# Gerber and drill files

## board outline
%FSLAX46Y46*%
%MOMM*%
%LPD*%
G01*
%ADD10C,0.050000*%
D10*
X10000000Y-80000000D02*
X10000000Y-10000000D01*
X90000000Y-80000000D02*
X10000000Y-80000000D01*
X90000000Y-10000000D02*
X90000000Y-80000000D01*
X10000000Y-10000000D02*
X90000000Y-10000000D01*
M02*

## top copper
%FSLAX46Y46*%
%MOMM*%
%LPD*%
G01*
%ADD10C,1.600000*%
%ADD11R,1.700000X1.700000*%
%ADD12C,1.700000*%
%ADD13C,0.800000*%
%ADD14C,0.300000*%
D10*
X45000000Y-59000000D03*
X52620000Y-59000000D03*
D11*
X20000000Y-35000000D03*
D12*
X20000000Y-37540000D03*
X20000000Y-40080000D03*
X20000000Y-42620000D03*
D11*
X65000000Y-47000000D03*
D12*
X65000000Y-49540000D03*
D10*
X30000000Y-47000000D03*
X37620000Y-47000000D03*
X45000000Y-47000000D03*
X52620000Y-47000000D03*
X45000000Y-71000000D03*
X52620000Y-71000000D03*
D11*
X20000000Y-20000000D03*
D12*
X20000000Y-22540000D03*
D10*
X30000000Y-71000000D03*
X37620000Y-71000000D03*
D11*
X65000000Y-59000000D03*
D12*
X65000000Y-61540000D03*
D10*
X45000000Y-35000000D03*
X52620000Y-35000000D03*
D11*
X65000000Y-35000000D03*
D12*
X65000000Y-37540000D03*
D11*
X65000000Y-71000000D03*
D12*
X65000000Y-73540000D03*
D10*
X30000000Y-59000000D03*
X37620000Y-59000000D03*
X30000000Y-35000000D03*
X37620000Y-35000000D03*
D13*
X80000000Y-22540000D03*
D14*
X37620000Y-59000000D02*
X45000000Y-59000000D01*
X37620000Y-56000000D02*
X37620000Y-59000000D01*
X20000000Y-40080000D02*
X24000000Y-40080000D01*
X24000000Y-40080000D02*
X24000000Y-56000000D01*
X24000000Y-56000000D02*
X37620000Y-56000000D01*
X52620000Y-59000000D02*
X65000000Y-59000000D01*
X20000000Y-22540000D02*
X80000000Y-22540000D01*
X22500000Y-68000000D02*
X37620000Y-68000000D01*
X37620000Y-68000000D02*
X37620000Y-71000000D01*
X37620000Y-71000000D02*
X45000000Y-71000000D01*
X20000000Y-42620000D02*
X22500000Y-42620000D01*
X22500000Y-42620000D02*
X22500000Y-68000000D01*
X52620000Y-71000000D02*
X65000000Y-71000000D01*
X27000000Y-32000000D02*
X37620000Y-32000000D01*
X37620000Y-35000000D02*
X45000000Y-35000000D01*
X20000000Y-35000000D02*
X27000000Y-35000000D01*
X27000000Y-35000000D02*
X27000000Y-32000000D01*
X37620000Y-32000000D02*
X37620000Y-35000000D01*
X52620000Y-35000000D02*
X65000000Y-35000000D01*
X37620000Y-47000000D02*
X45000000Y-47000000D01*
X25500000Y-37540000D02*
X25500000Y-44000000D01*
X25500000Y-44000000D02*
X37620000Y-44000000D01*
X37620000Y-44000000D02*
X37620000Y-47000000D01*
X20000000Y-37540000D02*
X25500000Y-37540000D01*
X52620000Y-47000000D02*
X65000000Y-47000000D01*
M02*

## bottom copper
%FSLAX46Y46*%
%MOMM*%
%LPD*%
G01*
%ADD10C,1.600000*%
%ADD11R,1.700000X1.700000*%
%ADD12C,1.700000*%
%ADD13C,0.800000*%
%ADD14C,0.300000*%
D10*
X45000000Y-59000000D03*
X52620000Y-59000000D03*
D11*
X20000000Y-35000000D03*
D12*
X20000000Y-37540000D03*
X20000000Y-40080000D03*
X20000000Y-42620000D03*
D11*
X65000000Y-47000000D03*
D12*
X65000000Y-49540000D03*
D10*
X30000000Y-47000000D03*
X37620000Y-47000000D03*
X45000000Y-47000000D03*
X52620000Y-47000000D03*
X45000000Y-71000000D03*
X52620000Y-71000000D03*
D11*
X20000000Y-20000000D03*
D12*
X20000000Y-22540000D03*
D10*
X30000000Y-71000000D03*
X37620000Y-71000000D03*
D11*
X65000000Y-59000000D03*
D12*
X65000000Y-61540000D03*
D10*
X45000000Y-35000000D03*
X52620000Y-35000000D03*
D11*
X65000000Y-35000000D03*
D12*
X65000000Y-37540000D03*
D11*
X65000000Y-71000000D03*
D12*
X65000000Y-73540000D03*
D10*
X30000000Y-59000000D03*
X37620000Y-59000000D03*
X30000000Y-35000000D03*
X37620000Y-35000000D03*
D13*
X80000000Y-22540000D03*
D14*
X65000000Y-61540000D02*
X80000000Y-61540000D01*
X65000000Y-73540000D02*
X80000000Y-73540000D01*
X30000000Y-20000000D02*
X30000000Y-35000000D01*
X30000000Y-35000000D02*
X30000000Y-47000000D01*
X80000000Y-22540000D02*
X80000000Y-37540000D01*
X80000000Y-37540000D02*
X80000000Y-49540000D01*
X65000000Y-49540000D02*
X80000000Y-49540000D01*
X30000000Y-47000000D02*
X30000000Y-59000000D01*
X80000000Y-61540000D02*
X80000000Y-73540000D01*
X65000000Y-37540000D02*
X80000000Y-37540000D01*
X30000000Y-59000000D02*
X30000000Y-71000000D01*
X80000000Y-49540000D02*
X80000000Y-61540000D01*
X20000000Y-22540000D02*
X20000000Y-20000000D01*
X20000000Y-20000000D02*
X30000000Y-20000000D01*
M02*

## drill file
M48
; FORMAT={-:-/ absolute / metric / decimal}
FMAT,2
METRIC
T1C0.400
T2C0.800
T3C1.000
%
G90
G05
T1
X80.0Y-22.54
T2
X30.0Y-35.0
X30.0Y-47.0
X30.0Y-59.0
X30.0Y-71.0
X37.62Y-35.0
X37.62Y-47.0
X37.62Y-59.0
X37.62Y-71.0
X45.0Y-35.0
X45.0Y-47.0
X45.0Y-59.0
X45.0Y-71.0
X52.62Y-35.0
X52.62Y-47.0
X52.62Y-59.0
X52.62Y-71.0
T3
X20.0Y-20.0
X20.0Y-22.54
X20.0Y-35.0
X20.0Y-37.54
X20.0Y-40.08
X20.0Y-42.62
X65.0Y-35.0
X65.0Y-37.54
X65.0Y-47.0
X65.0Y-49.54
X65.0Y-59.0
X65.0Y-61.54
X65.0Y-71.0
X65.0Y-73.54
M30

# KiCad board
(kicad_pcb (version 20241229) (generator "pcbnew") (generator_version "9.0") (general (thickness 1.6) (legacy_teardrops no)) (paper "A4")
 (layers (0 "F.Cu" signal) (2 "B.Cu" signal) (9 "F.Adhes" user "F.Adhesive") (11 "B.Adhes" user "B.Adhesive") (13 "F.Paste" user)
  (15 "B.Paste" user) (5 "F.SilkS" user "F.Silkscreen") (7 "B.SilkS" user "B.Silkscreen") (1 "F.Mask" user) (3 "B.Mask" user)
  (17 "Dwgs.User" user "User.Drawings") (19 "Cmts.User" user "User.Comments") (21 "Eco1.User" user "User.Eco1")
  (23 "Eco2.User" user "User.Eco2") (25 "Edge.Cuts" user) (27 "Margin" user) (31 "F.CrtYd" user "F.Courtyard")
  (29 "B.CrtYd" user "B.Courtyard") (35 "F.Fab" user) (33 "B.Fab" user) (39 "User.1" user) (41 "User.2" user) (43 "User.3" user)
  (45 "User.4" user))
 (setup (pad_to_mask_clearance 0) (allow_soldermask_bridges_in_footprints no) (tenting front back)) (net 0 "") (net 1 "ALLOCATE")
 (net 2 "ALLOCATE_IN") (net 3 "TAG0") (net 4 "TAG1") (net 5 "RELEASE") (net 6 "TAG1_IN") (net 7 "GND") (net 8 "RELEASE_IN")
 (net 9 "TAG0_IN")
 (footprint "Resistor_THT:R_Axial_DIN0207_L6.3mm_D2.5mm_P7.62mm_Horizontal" (layer "F.Cu") (at 45 59)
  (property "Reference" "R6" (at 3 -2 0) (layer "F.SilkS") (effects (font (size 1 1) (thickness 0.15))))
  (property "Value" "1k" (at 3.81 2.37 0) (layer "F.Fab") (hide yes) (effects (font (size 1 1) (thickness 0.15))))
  (pad "1" thru_hole circle (at 0 0) (size 1.6 1.6) (drill 0.8) (layers "*.Cu" "*.Mask") (remove_unused_layers no) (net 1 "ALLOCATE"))
  (pad "2" thru_hole circle (at 7.62 0) (size 1.6 1.6) (drill 0.8) (layers "*.Cu" "*.Mask") (remove_unused_layers no) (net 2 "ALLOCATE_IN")))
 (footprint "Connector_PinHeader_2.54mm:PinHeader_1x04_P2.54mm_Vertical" (layer "F.Cu") (at 20 35)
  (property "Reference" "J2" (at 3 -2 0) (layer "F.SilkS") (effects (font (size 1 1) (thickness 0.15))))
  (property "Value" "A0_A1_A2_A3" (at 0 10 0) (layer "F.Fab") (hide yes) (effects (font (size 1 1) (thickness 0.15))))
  (pad "1" thru_hole rect (at 0 0) (size 1.7 1.7) (drill 1) (layers "*.Cu" "*.Mask") (remove_unused_layers no) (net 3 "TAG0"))
  (pad "2" thru_hole circle (at 0 2.54) (size 1.7 1.7) (drill 1) (layers "*.Cu" "*.Mask") (remove_unused_layers no) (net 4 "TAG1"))
  (pad "3" thru_hole circle (at 0 5.08) (size 1.7 1.7) (drill 1) (layers "*.Cu" "*.Mask") (remove_unused_layers no) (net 1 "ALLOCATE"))
  (pad "4" thru_hole circle (at 0 7.62) (size 1.7 1.7) (drill 1) (layers "*.Cu" "*.Mask") (remove_unused_layers no) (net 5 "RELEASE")))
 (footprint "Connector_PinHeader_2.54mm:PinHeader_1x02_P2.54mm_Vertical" (layer "F.Cu") (at 65 47)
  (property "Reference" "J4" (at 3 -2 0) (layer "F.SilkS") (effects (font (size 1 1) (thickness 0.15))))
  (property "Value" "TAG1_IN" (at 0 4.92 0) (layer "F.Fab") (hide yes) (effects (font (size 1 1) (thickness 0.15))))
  (pad "1" thru_hole rect (at 0 0) (size 1.7 1.7) (drill 1) (layers "*.Cu" "*.Mask") (remove_unused_layers no) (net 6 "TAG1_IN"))
  (pad "2" thru_hole circle (at 0 2.54) (size 1.7 1.7) (drill 1) (layers "*.Cu" "*.Mask") (remove_unused_layers no) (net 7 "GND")))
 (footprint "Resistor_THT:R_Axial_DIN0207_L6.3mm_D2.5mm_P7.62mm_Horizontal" (layer "F.Cu") (at 30 47)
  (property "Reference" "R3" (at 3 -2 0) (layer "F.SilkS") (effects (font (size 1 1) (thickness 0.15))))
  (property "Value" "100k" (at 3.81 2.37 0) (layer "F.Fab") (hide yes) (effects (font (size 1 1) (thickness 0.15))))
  (pad "1" thru_hole circle (at 0 0) (size 1.6 1.6) (drill 0.8) (layers "*.Cu" "*.Mask") (remove_unused_layers no) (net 7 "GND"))
  (pad "2" thru_hole circle (at 7.62 0) (size 1.6 1.6) (drill 0.8) (layers "*.Cu" "*.Mask") (remove_unused_layers no) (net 4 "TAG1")))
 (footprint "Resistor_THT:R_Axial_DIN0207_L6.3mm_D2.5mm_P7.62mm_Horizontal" (layer "F.Cu") (at 45 47)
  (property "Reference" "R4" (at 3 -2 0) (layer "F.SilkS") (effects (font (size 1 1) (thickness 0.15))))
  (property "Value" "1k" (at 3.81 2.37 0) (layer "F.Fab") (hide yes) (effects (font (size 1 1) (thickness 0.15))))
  (pad "1" thru_hole circle (at 0 0) (size 1.6 1.6) (drill 0.8) (layers "*.Cu" "*.Mask") (remove_unused_layers no) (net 4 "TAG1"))
  (pad "2" thru_hole circle (at 7.62 0) (size 1.6 1.6) (drill 0.8) (layers "*.Cu" "*.Mask") (remove_unused_layers no) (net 6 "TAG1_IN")))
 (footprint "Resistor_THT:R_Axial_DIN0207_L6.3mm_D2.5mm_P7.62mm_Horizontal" (layer "F.Cu") (at 45 71)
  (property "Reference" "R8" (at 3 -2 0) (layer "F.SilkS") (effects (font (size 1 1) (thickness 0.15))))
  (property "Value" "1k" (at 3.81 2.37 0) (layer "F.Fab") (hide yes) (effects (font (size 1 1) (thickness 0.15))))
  (pad "1" thru_hole circle (at 0 0) (size 1.6 1.6) (drill 0.8) (layers "*.Cu" "*.Mask") (remove_unused_layers no) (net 5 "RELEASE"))
  (pad "2" thru_hole circle (at 7.62 0) (size 1.6 1.6) (drill 0.8) (layers "*.Cu" "*.Mask") (remove_unused_layers no) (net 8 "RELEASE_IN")))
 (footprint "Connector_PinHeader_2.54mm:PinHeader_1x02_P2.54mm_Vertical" (layer "F.Cu") (at 20 20)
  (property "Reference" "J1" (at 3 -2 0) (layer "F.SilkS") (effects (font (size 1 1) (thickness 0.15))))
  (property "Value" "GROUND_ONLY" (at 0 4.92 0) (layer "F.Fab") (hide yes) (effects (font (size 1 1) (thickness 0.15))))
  (pad "1" thru_hole rect (at 0 0) (size 1.7 1.7) (drill 1) (layers "*.Cu" "*.Mask") (remove_unused_layers no) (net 7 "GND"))
  (pad "2" thru_hole circle (at 0 2.54) (size 1.7 1.7) (drill 1) (layers "*.Cu" "*.Mask") (remove_unused_layers no) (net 7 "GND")))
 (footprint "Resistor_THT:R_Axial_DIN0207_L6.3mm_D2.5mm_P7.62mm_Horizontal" (layer "F.Cu") (at 30 71)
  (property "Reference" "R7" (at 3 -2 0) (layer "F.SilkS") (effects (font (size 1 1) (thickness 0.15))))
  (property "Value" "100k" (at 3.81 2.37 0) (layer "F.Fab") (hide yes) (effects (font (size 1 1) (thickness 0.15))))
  (pad "1" thru_hole circle (at 0 0) (size 1.6 1.6) (drill 0.8) (layers "*.Cu" "*.Mask") (remove_unused_layers no) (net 7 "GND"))
  (pad "2" thru_hole circle (at 7.62 0) (size 1.6 1.6) (drill 0.8) (layers "*.Cu" "*.Mask") (remove_unused_layers no) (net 5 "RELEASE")))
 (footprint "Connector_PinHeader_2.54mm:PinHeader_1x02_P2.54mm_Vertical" (layer "F.Cu") (at 65 59)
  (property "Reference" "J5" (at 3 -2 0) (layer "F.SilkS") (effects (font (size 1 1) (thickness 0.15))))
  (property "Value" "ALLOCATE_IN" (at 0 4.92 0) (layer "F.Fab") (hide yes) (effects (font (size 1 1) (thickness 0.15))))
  (pad "1" thru_hole rect (at 0 0) (size 1.7 1.7) (drill 1) (layers "*.Cu" "*.Mask") (remove_unused_layers no) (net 2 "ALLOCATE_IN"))
  (pad "2" thru_hole circle (at 0 2.54) (size 1.7 1.7) (drill 1) (layers "*.Cu" "*.Mask") (remove_unused_layers no) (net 7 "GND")))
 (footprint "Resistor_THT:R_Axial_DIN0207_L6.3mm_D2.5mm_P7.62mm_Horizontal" (layer "F.Cu") (at 45 35)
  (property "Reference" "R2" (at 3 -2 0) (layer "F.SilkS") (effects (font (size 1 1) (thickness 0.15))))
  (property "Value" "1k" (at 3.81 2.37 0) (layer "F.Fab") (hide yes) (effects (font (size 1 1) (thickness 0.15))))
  (pad "1" thru_hole circle (at 0 0) (size 1.6 1.6) (drill 0.8) (layers "*.Cu" "*.Mask") (remove_unused_layers no) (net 3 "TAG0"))
  (pad "2" thru_hole circle (at 7.62 0) (size 1.6 1.6) (drill 0.8) (layers "*.Cu" "*.Mask") (remove_unused_layers no) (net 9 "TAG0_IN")))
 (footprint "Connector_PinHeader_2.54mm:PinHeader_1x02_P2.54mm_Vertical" (layer "F.Cu") (at 65 35)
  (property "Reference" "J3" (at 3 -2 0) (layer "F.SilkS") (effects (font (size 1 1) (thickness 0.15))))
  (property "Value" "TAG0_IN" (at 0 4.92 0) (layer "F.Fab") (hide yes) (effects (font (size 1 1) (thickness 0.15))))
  (pad "1" thru_hole rect (at 0 0) (size 1.7 1.7) (drill 1) (layers "*.Cu" "*.Mask") (remove_unused_layers no) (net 9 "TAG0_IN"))
  (pad "2" thru_hole circle (at 0 2.54) (size 1.7 1.7) (drill 1) (layers "*.Cu" "*.Mask") (remove_unused_layers no) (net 7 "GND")))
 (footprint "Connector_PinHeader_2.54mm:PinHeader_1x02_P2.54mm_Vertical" (layer "F.Cu") (at 65 71)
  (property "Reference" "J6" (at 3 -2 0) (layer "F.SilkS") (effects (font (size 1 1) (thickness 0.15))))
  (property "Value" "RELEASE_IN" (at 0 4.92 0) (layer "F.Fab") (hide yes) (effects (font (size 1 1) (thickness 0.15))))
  (pad "1" thru_hole rect (at 0 0) (size 1.7 1.7) (drill 1) (layers "*.Cu" "*.Mask") (remove_unused_layers no) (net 8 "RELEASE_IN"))
  (pad "2" thru_hole circle (at 0 2.54) (size 1.7 1.7) (drill 1) (layers "*.Cu" "*.Mask") (remove_unused_layers no) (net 7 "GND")))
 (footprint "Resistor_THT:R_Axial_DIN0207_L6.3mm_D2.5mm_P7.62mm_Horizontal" (layer "F.Cu") (at 30 59)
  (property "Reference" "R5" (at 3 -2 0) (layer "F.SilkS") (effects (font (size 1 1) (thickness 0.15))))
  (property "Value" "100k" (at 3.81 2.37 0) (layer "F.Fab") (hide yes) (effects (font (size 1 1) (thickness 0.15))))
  (pad "1" thru_hole circle (at 0 0) (size 1.6 1.6) (drill 0.8) (layers "*.Cu" "*.Mask") (remove_unused_layers no) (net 7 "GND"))
  (pad "2" thru_hole circle (at 7.62 0) (size 1.6 1.6) (drill 0.8) (layers "*.Cu" "*.Mask") (remove_unused_layers no) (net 1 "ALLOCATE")))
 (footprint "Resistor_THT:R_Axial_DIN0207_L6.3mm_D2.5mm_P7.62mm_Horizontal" (layer "F.Cu") (at 30 35)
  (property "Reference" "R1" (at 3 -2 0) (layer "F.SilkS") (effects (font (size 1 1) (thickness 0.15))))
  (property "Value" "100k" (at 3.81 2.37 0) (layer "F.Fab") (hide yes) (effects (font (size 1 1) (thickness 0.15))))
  (pad "1" thru_hole circle (at 0 0) (size 1.6 1.6) (drill 0.8) (layers "*.Cu" "*.Mask") (remove_unused_layers no) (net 7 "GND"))
  (pad "2" thru_hole circle (at 7.62 0) (size 1.6 1.6) (drill 0.8) (layers "*.Cu" "*.Mask") (remove_unused_layers no) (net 3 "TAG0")))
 (gr_line (start 10 80) (end 10 10) (stroke (width 0.05) (type default)) (layer "Edge.Cuts"))
 (gr_line (start 90 80) (end 10 80) (stroke (width 0.05) (type default)) (layer "Edge.Cuts"))
 (gr_line (start 90 10) (end 90 80) (stroke (width 0.05) (type default)) (layer "Edge.Cuts"))
 (gr_line (start 10 10) (end 90 10) (stroke (width 0.05) (type default)) (layer "Edge.Cuts"))
 (segment (start 37.62 59) (end 45 59) (width 0.3) (layer "F.Cu") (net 1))
 (segment (start 37.62 56) (end 37.62 59) (width 0.3) (layer "F.Cu") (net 1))
 (segment (start 20 40.08) (end 24 40.08) (width 0.3) (layer "F.Cu") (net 1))
 (segment (start 24 40.08) (end 24 56) (width 0.3) (layer "F.Cu") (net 1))
 (segment (start 24 56) (end 37.62 56) (width 0.3) (layer "F.Cu") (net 1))
 (segment (start 52.62 59) (end 65 59) (width 0.3) (layer "F.Cu") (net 2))
 (segment (start 20 22.54) (end 80 22.54) (width 0.3) (layer "F.Cu") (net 7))
 (via (at 80 22.54) (size 0.8) (drill 0.4) (layers "F.Cu" "B.Cu") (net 7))
 (segment (start 65 61.54) (end 80 61.54) (width 0.3) (layer "B.Cu") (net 7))
 (segment (start 65 73.54) (end 80 73.54) (width 0.3) (layer "B.Cu") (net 7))
 (segment (start 30 20) (end 30 35) (width 0.3) (layer "B.Cu") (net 7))
 (segment (start 30 35) (end 30 47) (width 0.3) (layer "B.Cu") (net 7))
 (segment (start 80 22.54) (end 80 37.54) (width 0.3) (layer "B.Cu") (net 7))
 (segment (start 80 37.54) (end 80 49.54) (width 0.3) (layer "B.Cu") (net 7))
 (segment (start 65 49.54) (end 80 49.54) (width 0.3) (layer "B.Cu") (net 7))
 (segment (start 30 47) (end 30 59) (width 0.3) (layer "B.Cu") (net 7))
 (segment (start 80 61.54) (end 80 73.54) (width 0.3) (layer "B.Cu") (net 7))
 (segment (start 65 37.54) (end 80 37.54) (width 0.3) (layer "B.Cu") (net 7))
 (segment (start 30 59) (end 30 71) (width 0.3) (layer "B.Cu") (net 7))
 (segment (start 80 49.54) (end 80 61.54) (width 0.3) (layer "B.Cu") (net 7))
 (segment (start 20 22.54) (end 20 20) (width 0.3) (layer "B.Cu") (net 7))
 (segment (start 20 20) (end 30 20) (width 0.3) (layer "B.Cu") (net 7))
 (segment (start 22.5 68) (end 37.62 68) (width 0.3) (layer "F.Cu") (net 5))
 (segment (start 37.62 68) (end 37.62 71) (width 0.3) (layer "F.Cu") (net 5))
 (segment (start 37.62 71) (end 45 71) (width 0.3) (layer "F.Cu") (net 5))
 (segment (start 20 42.62) (end 22.5 42.62) (width 0.3) (layer "F.Cu") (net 5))
 (segment (start 22.5 42.62) (end 22.5 68) (width 0.3) (layer "F.Cu") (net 5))
 (segment (start 52.62 71) (end 65 71) (width 0.3) (layer "F.Cu") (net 8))
 (segment (start 27 32) (end 37.62 32) (width 0.3) (layer "F.Cu") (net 3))
 (segment (start 37.62 35) (end 45 35) (width 0.3) (layer "F.Cu") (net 3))
 (segment (start 20 35) (end 27 35) (width 0.3) (layer "F.Cu") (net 3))
 (segment (start 27 35) (end 27 32) (width 0.3) (layer "F.Cu") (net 3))
 (segment (start 37.62 32) (end 37.62 35) (width 0.3) (layer "F.Cu") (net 3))
 (segment (start 52.62 35) (end 65 35) (width 0.3) (layer "F.Cu") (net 9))
 (segment (start 37.62 47) (end 45 47) (width 0.3) (layer "F.Cu") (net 4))
 (segment (start 25.5 37.54) (end 25.5 44) (width 0.3) (layer "F.Cu") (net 4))
 (segment (start 25.5 44) (end 37.62 44) (width 0.3) (layer "F.Cu") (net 4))
 (segment (start 37.62 44) (end 37.62 47) (width 0.3) (layer "F.Cu") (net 4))
 (segment (start 20 37.54) (end 25.5 37.54) (width 0.3) (layer "F.Cu") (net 4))
 (segment (start 52.62 47) (end 65 47) (width 0.3) (layer "F.Cu") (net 6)))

